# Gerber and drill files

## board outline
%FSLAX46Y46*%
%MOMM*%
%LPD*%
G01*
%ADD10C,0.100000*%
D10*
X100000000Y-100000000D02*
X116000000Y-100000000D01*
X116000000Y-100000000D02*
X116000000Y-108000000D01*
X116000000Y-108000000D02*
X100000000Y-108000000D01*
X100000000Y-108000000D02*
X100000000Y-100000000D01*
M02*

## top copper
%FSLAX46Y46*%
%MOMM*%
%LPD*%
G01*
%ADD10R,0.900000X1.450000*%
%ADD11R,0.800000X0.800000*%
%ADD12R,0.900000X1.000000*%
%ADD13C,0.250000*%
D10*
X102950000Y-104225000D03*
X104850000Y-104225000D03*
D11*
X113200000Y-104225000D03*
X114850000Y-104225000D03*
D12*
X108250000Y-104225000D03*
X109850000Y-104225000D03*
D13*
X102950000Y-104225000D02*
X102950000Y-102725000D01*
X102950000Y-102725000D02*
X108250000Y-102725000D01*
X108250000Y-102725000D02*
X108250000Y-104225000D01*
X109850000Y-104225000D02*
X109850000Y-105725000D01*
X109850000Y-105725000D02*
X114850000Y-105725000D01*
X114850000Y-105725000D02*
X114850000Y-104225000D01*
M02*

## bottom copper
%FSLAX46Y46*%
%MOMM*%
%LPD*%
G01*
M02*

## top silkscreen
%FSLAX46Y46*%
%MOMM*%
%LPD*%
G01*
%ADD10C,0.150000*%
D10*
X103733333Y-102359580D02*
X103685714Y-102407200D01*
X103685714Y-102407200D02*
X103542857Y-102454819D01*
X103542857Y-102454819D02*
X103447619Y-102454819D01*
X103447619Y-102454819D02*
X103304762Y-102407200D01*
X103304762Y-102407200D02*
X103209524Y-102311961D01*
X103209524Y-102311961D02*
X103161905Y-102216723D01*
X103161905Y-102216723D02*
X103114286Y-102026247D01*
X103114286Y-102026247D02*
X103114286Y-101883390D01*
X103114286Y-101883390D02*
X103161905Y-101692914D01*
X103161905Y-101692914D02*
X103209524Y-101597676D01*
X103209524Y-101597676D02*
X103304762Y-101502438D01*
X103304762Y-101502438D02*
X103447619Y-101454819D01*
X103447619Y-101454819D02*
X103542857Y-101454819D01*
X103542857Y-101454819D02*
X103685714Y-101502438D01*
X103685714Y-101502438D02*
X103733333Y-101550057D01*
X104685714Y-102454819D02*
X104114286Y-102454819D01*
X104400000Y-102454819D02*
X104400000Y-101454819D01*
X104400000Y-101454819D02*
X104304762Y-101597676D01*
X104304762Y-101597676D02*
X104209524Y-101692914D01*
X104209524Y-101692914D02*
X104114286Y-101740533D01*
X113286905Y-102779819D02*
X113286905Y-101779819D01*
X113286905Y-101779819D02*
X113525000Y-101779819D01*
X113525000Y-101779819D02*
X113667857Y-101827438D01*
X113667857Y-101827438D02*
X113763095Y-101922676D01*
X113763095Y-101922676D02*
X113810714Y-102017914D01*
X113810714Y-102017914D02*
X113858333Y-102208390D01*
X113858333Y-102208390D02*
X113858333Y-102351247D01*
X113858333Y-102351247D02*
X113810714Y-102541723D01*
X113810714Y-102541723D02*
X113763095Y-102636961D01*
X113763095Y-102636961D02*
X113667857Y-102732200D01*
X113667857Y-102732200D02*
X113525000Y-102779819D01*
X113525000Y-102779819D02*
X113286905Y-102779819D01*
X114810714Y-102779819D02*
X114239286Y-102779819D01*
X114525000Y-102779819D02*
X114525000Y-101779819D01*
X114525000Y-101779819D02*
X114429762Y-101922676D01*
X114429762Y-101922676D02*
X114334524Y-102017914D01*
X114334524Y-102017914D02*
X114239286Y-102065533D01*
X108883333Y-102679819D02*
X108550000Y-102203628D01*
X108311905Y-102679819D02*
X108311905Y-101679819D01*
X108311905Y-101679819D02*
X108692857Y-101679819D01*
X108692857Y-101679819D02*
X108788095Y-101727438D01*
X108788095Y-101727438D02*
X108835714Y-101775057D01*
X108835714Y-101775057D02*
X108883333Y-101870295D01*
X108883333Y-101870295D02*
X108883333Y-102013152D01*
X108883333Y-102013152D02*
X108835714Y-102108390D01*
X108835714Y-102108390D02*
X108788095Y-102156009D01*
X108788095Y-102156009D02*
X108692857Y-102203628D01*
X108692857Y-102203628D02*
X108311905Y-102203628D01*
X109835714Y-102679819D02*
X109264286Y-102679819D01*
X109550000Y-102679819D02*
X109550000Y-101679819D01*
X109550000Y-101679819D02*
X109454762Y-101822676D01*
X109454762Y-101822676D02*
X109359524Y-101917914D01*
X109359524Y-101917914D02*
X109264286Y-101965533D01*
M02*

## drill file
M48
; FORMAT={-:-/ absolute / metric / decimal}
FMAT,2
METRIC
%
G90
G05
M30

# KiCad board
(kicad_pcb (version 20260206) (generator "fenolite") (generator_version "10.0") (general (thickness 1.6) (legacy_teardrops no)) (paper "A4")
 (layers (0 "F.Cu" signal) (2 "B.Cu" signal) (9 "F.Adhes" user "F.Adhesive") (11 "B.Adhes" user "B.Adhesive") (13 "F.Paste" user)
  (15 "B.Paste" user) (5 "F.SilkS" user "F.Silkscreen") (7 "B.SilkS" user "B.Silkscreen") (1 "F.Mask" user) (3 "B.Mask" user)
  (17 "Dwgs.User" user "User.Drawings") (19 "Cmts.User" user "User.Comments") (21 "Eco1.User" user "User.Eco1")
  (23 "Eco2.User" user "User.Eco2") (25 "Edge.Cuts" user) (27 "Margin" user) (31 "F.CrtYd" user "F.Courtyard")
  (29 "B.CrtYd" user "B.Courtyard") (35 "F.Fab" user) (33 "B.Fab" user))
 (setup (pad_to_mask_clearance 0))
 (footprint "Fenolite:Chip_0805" (layer "F.Cu") (at 103.9 104.225)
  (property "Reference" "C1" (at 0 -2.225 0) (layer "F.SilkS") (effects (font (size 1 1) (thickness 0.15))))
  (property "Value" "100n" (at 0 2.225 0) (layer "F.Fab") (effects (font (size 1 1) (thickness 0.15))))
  (pad "1" smd rect (at -0.95 0) (size 0.9 1.45) (layers "F.Cu" "F.Paste" "F.Mask") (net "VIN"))
  (pad "2" smd rect (at 0.95 0) (size 0.9 1.45) (layers "F.Cu" "F.Paste" "F.Mask") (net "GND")))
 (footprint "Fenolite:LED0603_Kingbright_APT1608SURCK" (layer "F.Cu") (at 114.025 104.225)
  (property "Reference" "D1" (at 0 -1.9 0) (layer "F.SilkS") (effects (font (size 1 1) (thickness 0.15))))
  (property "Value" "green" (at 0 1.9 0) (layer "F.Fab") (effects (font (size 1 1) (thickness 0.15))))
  (pad "1" smd rect (at -0.825 0) (size 0.8 0.8) (layers "F.Cu" "F.Paste" "F.Mask") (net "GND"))
  (pad "2" smd rect (at 0.825 0) (size 0.8 0.8) (layers "F.Cu" "F.Paste" "F.Mask") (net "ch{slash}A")))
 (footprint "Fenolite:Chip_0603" (layer "F.Cu") (at 109.05 104.225)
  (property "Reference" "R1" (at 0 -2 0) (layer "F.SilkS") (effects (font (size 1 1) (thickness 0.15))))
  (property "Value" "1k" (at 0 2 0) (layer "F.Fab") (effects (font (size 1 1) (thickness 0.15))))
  (pad "1" smd rect (at -0.8 0) (size 0.9 1) (layers "F.Cu" "F.Paste" "F.Mask") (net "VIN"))
  (pad "2" smd rect (at 0.8 0) (size 0.9 1) (layers "F.Cu" "F.Paste" "F.Mask") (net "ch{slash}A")))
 (gr_line (start 100 100) (end 116 100) (stroke (width 0.1) (type solid)) (layer "Edge.Cuts"))
 (gr_line (start 116 100) (end 116 108) (stroke (width 0.1) (type solid)) (layer "Edge.Cuts"))
 (gr_line (start 116 108) (end 100 108) (stroke (width 0.1) (type solid)) (layer "Edge.Cuts"))
 (gr_line (start 100 108) (end 100 100) (stroke (width 0.1) (type solid)) (layer "Edge.Cuts"))
 (segment (start 102.95 104.225) (end 102.95 102.725) (width 0.25) (layer "F.Cu") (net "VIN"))
 (segment (start 102.95 102.725) (end 108.25 102.725) (width 0.25) (layer "F.Cu") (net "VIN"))
 (segment (start 108.25 102.725) (end 108.25 104.225) (width 0.25) (layer "F.Cu") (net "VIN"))
 (segment (start 109.85 104.225) (end 109.85 105.725) (width 0.25) (layer "F.Cu") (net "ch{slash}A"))
 (segment (start 109.85 105.725) (end 114.85 105.725) (width 0.25) (layer "F.Cu") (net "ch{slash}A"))
 (segment (start 114.85 105.725) (end 114.85 104.225) (width 0.25) (layer "F.Cu") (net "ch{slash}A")))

